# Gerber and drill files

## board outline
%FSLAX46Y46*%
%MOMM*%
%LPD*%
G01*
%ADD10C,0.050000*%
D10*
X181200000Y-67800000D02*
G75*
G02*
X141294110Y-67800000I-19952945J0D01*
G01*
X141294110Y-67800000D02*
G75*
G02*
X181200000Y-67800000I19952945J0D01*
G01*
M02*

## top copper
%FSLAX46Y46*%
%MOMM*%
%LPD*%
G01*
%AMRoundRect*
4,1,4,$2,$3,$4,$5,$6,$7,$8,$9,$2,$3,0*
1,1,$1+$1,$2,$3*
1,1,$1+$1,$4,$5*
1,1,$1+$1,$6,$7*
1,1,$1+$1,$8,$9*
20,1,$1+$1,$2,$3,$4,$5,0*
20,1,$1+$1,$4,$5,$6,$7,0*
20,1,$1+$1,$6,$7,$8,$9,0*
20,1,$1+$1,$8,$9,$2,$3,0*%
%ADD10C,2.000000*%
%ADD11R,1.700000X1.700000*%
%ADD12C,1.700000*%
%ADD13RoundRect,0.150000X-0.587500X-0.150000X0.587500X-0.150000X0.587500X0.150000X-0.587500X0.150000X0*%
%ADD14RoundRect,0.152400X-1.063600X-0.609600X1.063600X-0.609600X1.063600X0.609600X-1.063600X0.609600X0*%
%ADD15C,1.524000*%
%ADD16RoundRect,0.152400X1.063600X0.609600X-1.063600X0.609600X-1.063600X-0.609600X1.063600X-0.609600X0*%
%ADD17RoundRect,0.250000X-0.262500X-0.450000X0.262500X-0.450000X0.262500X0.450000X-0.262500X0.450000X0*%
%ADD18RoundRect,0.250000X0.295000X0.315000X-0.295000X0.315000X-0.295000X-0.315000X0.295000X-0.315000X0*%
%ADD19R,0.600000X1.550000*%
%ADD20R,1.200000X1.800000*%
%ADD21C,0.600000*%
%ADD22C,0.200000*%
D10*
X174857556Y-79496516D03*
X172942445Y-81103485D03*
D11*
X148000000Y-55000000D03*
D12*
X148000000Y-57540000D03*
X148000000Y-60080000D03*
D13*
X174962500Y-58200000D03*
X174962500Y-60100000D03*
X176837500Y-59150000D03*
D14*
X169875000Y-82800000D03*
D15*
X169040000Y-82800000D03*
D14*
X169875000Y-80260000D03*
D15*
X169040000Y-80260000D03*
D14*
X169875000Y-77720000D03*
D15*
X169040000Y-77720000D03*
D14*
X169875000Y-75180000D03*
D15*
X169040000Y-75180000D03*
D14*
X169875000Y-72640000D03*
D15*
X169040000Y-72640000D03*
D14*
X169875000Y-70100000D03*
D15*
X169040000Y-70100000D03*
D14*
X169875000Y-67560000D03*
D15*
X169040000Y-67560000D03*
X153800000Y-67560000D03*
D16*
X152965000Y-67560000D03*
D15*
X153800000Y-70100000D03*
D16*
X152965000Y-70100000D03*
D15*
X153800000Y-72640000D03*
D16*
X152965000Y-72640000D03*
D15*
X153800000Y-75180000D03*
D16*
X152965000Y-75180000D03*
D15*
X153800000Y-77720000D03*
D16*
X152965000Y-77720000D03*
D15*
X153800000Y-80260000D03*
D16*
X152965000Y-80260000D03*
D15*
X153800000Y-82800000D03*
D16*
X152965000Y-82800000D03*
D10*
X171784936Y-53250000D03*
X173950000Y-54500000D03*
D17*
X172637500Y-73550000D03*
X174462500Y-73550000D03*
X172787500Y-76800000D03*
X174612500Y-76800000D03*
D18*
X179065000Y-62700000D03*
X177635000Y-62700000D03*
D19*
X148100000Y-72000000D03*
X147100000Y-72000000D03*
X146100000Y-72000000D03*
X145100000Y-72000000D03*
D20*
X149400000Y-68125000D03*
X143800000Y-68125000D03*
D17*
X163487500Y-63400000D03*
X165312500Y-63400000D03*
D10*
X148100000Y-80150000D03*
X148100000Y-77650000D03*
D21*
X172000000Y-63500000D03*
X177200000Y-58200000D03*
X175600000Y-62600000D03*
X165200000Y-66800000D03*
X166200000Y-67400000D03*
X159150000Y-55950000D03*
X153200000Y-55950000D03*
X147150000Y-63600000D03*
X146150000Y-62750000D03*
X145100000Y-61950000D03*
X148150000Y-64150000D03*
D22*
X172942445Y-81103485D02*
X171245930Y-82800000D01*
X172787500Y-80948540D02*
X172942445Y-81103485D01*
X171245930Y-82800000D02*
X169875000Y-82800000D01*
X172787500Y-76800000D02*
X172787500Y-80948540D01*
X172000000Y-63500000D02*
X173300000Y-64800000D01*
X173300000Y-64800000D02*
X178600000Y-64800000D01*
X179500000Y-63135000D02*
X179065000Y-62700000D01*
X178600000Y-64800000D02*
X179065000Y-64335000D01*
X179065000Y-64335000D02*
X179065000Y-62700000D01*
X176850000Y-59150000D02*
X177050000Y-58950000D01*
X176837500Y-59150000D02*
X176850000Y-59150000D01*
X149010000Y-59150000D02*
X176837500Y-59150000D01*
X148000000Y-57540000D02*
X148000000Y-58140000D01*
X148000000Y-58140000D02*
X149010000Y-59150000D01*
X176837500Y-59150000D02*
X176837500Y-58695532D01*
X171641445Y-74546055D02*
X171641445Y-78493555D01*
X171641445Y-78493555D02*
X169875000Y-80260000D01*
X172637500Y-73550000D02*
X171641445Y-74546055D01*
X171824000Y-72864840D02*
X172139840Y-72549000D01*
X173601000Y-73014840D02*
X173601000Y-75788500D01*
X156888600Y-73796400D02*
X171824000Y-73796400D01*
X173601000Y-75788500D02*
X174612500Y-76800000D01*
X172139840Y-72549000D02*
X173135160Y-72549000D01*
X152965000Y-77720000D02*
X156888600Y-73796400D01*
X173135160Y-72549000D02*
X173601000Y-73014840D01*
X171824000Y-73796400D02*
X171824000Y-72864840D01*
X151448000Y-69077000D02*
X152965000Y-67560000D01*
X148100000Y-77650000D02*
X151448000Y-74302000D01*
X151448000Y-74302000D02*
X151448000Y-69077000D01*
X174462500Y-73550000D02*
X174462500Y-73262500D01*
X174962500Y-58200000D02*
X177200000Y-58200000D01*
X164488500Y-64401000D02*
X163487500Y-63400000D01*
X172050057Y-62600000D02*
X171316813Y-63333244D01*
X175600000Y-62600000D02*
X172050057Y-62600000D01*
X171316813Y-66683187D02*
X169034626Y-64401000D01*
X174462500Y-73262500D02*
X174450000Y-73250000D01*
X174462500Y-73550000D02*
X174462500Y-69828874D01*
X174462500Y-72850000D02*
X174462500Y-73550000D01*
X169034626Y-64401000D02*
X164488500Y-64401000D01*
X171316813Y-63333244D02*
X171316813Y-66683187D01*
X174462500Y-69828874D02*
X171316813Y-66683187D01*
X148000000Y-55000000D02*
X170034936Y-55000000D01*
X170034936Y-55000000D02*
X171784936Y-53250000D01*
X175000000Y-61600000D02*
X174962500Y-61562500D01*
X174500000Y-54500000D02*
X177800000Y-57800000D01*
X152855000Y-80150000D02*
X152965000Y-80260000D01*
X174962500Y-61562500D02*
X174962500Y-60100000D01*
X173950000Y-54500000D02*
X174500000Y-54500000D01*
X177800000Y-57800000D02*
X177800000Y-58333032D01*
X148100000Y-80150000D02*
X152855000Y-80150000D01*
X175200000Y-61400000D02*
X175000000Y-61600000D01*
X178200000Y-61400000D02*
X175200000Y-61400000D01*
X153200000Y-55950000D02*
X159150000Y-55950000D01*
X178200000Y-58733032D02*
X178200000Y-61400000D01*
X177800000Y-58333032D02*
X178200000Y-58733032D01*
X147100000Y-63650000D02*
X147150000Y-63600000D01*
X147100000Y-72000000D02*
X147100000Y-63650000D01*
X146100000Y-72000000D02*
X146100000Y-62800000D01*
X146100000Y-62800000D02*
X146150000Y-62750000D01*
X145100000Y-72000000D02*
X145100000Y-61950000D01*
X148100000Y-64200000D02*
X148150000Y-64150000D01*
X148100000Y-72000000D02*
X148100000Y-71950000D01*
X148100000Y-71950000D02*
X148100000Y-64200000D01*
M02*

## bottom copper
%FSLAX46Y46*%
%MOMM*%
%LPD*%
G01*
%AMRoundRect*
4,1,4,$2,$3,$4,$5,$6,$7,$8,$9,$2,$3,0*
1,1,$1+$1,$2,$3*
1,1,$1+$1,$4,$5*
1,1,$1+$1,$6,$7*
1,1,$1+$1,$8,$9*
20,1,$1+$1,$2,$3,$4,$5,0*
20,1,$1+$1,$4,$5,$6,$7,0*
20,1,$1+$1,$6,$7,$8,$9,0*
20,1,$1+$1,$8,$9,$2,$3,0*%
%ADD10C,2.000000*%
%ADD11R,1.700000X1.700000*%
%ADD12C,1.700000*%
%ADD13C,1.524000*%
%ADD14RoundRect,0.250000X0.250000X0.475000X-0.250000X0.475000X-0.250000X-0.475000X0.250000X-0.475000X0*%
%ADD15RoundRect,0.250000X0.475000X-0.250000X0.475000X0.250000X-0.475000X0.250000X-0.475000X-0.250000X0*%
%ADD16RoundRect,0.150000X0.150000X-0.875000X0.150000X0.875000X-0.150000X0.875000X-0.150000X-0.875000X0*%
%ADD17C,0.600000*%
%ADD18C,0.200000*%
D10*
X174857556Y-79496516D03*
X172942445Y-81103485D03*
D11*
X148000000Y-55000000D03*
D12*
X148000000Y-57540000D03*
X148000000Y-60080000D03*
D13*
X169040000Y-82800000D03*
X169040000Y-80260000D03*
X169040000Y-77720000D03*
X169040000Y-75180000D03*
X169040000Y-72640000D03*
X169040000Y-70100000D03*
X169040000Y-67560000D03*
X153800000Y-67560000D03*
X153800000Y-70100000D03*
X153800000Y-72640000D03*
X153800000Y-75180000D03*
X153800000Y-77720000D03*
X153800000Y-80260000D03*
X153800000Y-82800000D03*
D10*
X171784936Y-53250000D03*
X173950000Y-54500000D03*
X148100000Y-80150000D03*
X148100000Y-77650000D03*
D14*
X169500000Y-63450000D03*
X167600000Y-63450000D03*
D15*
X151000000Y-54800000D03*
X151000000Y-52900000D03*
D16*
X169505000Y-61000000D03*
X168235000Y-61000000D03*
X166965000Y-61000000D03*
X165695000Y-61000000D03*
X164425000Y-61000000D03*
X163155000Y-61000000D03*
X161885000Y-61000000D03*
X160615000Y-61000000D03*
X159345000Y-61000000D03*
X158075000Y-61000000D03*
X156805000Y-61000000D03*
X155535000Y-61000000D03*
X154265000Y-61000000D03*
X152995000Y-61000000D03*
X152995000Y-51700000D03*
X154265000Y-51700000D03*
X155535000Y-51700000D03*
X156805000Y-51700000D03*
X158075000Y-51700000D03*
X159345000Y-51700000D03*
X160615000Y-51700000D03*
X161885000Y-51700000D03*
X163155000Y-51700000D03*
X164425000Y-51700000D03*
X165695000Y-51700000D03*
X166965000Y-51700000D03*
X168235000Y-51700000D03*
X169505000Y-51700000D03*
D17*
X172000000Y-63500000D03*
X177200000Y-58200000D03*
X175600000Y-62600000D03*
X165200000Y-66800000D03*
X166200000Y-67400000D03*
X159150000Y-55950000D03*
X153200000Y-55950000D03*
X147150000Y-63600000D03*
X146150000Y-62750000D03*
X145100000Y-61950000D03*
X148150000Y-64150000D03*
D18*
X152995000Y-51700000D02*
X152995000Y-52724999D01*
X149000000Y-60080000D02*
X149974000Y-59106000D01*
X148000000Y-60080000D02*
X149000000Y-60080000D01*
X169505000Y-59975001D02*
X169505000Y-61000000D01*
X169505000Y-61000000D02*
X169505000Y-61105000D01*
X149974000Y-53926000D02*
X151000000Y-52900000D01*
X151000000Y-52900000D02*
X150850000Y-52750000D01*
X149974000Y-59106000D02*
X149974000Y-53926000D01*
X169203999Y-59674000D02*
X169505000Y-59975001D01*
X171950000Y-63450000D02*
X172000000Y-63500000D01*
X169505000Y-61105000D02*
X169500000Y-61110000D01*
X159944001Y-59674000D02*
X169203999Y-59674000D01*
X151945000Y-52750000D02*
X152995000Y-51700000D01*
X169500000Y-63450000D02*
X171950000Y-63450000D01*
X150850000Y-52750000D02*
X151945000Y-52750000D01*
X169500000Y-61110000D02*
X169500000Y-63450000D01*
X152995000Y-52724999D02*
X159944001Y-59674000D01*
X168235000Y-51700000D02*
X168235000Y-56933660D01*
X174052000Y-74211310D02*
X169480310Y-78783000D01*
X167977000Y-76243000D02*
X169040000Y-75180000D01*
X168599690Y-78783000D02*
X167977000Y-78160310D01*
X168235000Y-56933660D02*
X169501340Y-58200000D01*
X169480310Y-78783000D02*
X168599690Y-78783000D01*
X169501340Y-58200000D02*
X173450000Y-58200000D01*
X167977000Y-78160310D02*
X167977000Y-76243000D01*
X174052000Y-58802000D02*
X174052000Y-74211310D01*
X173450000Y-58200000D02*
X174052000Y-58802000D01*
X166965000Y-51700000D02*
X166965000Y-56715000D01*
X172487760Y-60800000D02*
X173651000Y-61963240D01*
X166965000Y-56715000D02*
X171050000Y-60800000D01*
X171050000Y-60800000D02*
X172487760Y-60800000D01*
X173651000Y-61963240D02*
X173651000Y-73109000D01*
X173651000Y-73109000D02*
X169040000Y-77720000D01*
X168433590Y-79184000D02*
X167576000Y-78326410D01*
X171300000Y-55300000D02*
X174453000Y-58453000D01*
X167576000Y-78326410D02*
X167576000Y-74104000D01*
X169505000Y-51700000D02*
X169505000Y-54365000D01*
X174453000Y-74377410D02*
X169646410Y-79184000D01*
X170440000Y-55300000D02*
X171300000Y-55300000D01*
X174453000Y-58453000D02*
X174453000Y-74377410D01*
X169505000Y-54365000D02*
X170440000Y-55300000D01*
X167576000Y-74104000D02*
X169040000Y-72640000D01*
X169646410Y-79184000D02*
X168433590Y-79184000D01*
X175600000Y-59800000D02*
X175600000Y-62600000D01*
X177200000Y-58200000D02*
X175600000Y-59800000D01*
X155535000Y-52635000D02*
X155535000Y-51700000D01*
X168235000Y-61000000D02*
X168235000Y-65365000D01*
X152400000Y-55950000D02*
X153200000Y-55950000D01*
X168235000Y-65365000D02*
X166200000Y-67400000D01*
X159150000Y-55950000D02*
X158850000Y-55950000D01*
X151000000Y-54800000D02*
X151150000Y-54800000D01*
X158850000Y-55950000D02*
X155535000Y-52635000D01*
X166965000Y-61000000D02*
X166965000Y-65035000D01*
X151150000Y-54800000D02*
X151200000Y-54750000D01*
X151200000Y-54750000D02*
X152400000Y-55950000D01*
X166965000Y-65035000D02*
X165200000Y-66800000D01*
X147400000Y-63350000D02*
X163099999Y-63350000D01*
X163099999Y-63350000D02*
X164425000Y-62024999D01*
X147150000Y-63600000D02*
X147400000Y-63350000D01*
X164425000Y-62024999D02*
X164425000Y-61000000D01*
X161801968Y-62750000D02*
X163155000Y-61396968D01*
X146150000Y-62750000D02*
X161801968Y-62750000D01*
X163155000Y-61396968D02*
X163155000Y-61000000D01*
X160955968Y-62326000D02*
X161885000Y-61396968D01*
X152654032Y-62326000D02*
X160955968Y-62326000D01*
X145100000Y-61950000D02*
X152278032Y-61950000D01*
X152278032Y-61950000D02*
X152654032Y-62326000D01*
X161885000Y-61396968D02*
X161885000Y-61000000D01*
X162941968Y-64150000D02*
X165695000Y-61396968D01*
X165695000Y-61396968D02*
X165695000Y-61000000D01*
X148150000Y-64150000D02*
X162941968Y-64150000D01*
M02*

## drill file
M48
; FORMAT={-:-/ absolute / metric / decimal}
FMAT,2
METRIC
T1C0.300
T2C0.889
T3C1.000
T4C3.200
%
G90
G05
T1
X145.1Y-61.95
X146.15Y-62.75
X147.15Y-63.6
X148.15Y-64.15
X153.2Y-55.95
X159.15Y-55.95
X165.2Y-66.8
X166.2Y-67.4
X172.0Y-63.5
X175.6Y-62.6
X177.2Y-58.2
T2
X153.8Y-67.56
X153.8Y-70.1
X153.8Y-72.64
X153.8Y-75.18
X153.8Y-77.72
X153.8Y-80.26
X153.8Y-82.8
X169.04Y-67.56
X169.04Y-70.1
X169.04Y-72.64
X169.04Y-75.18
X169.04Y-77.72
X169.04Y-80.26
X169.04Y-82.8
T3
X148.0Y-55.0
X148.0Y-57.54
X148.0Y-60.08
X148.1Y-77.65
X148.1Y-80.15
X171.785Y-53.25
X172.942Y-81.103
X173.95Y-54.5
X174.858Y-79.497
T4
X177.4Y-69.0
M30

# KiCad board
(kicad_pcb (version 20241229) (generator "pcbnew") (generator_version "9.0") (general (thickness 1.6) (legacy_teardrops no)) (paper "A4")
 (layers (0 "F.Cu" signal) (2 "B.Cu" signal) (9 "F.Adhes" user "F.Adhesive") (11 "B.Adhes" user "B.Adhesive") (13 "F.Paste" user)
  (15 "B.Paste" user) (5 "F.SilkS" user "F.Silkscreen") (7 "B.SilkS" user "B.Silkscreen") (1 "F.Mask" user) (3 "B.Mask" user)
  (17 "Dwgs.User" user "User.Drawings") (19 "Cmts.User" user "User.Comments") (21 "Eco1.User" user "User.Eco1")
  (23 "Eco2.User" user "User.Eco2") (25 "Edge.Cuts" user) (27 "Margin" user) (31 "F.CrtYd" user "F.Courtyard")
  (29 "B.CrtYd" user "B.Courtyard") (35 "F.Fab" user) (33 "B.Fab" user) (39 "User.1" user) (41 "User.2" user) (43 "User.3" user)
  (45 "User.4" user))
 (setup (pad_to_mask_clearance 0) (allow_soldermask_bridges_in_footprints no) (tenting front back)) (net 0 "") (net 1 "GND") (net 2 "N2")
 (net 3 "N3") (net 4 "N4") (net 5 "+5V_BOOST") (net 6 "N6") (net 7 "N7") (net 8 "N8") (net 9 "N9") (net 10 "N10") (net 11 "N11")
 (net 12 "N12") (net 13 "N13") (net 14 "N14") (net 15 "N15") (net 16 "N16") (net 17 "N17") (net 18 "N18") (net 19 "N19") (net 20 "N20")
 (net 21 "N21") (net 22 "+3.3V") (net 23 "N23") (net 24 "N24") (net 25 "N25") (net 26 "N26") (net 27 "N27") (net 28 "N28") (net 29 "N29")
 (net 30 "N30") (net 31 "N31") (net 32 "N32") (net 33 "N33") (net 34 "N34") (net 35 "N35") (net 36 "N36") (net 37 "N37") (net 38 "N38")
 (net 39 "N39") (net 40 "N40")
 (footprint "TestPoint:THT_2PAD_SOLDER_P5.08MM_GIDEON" (layer "F.Cu") (at 174.857556 79.496516 -140)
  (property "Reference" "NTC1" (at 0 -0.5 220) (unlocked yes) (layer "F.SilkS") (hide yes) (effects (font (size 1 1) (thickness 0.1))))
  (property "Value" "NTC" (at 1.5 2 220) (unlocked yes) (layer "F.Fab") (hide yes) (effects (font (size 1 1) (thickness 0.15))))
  (pad "1" thru_hole circle (at 0 0 220) (size 2 2) (drill 1) (layers "*.Cu" "*.Mask") (remove_unused_layers no) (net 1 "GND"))
  (pad "2" thru_hole circle (at 2.5 0 220) (size 2 2) (drill 1) (layers "*.Cu" "*.Mask") (remove_unused_layers no) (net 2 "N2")))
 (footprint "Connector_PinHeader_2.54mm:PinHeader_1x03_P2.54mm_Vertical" (layer "F.Cu") (at 148 55)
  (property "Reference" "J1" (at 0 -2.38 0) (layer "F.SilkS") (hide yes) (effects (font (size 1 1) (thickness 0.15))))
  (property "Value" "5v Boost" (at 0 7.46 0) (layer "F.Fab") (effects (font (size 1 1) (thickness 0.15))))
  (pad "1" thru_hole rect (at 0 0) (size 1.7 1.7) (drill 1) (layers "*.Cu" "*.Mask") (remove_unused_layers no) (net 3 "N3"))
  (pad "2" thru_hole circle (at 0 2.54) (size 1.7 1.7) (drill 1) (layers "*.Cu" "*.Mask") (remove_unused_layers no) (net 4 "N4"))
  (pad "3" thru_hole circle (at 0 5.08) (size 1.7 1.7) (drill 1) (layers "*.Cu" "*.Mask") (remove_unused_layers no) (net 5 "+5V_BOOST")))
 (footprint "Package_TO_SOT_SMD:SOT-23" (layer "F.Cu") (at 175.9 59.15)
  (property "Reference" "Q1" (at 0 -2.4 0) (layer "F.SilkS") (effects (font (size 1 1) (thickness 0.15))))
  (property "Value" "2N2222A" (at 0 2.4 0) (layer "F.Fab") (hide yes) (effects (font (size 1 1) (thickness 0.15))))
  (pad "1" smd roundrect (at -0.9375 -0.95) (size 1.475 0.6) (layers "F.Cu" "F.Mask" "F.Paste") (roundrect_rratio 0.25) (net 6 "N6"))
  (pad "2" smd roundrect (at -0.9375 0.95) (size 1.475 0.6) (layers "F.Cu" "F.Mask" "F.Paste") (roundrect_rratio 0.25) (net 1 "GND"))
  (pad "3" smd roundrect (at 0.9375 0) (size 1.475 0.6) (layers "F.Cu" "F.Mask" "F.Paste") (roundrect_rratio 0.25) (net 4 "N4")))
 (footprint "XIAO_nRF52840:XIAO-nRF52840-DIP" (layer "F.Cu") (at 161.42 75.18 180)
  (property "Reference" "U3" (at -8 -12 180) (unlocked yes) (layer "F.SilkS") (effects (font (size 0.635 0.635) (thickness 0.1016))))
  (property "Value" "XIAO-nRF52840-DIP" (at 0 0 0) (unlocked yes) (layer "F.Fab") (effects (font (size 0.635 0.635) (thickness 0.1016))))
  (pad "1" smd roundrect (at -8.455 -7.62) (size 2.432 1.524) (layers "F.Cu" "F.Mask") (roundrect_rratio 0.1) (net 2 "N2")
   (thermal_bridge_angle 45))
  (pad "1" thru_hole circle (at -7.62 -7.62) (size 1.524 1.524) (drill 0.889) (layers "*.Cu" "*.Mask") (remove_unused_layers no)
   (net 2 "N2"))
  (pad "2" smd roundrect (at -8.455 -5.08) (size 2.432 1.524) (layers "F.Cu" "F.Mask") (roundrect_rratio 0.1) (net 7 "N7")
   (thermal_bridge_angle 45))
  (pad "2" thru_hole circle (at -7.62 -5.08) (size 1.524 1.524) (drill 0.889) (layers "*.Cu" "*.Mask") (remove_unused_layers no)
   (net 7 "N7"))
  (pad "3" smd roundrect (at -8.455 -2.54) (size 2.432 1.524) (layers "F.Cu" "F.Mask") (roundrect_rratio 0.1) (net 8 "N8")
   (thermal_bridge_angle 45))
  (pad "3" thru_hole circle (at -7.62 -2.54) (size 1.524 1.524) (drill 0.889) (layers "*.Cu" "*.Mask") (remove_unused_layers no)
   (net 8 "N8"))
  (pad "4" smd roundrect (at -8.455 0) (size 2.432 1.524) (layers "F.Cu" "F.Mask") (roundrect_rratio 0.1) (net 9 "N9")
   (thermal_bridge_angle 45))
  (pad "4" thru_hole circle (at -7.62 0) (size 1.524 1.524) (drill 0.889) (layers "*.Cu" "*.Mask") (remove_unused_layers no) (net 9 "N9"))
  (pad "5" smd roundrect (at -8.455 2.54) (size 2.432 1.524) (layers "F.Cu" "F.Mask") (roundrect_rratio 0.1) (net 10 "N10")
   (thermal_bridge_angle 45))
  (pad "5" thru_hole circle (at -7.62 2.54) (size 1.524 1.524) (drill 0.889) (layers "*.Cu" "*.Mask") (remove_unused_layers no)
   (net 10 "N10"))
  (pad "6" smd roundrect (at -8.455 5.08) (size 2.432 1.524) (layers "F.Cu" "F.Mask") (roundrect_rratio 0.1) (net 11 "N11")
   (thermal_bridge_angle 45))
  (pad "6" thru_hole circle (at -7.62 5.08) (size 1.524 1.524) (drill 0.889) (layers "*.Cu" "*.Mask") (remove_unused_layers no)
   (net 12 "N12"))
  (pad "7" smd roundrect (at -8.455 7.62) (size 2.432 1.524) (layers "F.Cu" "F.Mask") (roundrect_rratio 0.1) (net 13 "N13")
   (thermal_bridge_angle 45))
  (pad "7" thru_hole circle (at -7.62 7.62) (size 1.524 1.524) (drill 0.889) (layers "*.Cu" "*.Mask") (remove_unused_layers no)
   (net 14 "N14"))
  (pad "8" thru_hole circle (at 7.62 7.62 180) (size 1.524 1.524) (drill 0.889) (layers "*.Cu" "*.Mask") (remove_unused_layers no)
   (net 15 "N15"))
  (pad "8" smd roundrect (at 8.455 7.62 180) (size 2.432 1.524) (layers "F.Cu" "F.Mask") (roundrect_rratio 0.1) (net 15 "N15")
   (thermal_bridge_angle 45))
  (pad "9" thru_hole circle (at 7.62 5.08 180) (size 1.524 1.524) (drill 0.889) (layers "*.Cu" "*.Mask") (remove_unused_layers no)
   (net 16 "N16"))
  (pad "9" smd roundrect (at 8.455 5.08 180) (size 2.432 1.524) (layers "F.Cu" "F.Mask") (roundrect_rratio 0.1) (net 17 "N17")
   (thermal_bridge_angle 45))
  (pad "10" thru_hole circle (at 7.62 2.54 180) (size 1.524 1.524) (drill 0.889) (layers "*.Cu" "*.Mask") (remove_unused_layers no)
   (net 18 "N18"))
  (pad "10" smd roundrect (at 8.455 2.54 180) (size 2.432 1.524) (layers "F.Cu" "F.Mask") (roundrect_rratio 0.1) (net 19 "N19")
   (thermal_bridge_angle 45))
  (pad "11" thru_hole circle (at 7.62 0 180) (size 1.524 1.524) (drill 0.889) (layers "*.Cu" "*.Mask") (remove_unused_layers no)
   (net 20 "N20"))
  (pad "11" smd roundrect (at 8.455 0 180) (size 2.432 1.524) (layers "F.Cu" "F.Mask") (roundrect_rratio 0.1) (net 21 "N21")
   (thermal_bridge_angle 45))
  (pad "12" thru_hole circle (at 7.62 -2.54 180) (size 1.524 1.524) (drill 0.889) (layers "*.Cu" "*.Mask") (remove_unused_layers no)
   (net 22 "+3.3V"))
  (pad "12" smd roundrect (at 8.455 -2.54 180) (size 2.432 1.524) (layers "F.Cu" "F.Mask") (roundrect_rratio 0.1) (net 22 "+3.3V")
   (thermal_bridge_angle 45))
  (pad "13" thru_hole circle (at 7.62 -5.08 180) (size 1.524 1.524) (drill 0.889) (layers "*.Cu" "*.Mask") (remove_unused_layers no)
   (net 1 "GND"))
  (pad "13" smd roundrect (at 8.455 -5.08 180) (size 2.432 1.524) (layers "F.Cu" "F.Mask") (roundrect_rratio 0.1) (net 1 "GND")
   (thermal_bridge_angle 45))
  (pad "14" thru_hole circle (at 7.62 -7.62 180) (size 1.524 1.524) (drill 0.889) (layers "*.Cu" "*.Mask") (remove_unused_layers no)
   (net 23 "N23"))
  (pad "14" smd roundrect (at 8.455 -7.62 180) (size 2.432 1.524) (layers "F.Cu" "F.Mask") (roundrect_rratio 0.1) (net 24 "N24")
   (thermal_bridge_angle 45)))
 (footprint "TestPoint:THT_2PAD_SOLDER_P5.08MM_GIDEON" (layer "F.Cu") (at 171.784936 53.25 -30)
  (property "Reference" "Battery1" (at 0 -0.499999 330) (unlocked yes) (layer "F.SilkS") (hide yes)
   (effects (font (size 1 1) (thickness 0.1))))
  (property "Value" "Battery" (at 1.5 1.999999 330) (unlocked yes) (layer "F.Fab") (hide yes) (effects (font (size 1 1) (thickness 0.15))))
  (pad "1" thru_hole circle (at 0 0 330) (size 2 2) (drill 1) (layers "*.Cu" "*.Mask") (remove_unused_layers no) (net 3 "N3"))
  (pad "2" thru_hole circle (at 2.5 0 330) (size 2 2) (drill 1) (layers "*.Cu" "*.Mask") (remove_unused_layers no) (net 1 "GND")))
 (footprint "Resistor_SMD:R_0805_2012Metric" (layer "F.Cu") (at 173.55 73.55)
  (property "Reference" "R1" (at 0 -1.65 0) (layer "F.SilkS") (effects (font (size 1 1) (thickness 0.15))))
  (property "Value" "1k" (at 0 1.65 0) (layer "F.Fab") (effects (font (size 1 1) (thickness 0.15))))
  (pad "1" smd roundrect (at -0.9125 0) (size 1.025 1.4) (layers "F.Cu" "F.Mask" "F.Paste") (roundrect_rratio 0.243902) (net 7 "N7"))
  (pad "2" smd roundrect (at 0.9125 0) (size 1.025 1.4) (layers "F.Cu" "F.Mask" "F.Paste") (roundrect_rratio 0.243902) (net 6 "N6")))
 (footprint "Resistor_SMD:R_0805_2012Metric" (layer "F.Cu") (at 173.7 76.8)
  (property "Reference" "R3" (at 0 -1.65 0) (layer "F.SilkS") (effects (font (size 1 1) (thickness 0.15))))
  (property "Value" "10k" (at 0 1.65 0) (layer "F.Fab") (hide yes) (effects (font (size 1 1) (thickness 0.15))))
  (pad "1" smd roundrect (at -0.9125 0) (size 1.025 1.4) (layers "F.Cu" "F.Mask" "F.Paste") (roundrect_rratio 0.243902) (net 2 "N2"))
  (pad "2" smd roundrect (at 0.9125 0) (size 1.025 1.4) (layers "F.Cu" "F.Mask" "F.Paste") (roundrect_rratio 0.243902) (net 22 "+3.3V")))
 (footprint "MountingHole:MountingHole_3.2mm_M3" (layer "F.Cu") (at 177.4 69)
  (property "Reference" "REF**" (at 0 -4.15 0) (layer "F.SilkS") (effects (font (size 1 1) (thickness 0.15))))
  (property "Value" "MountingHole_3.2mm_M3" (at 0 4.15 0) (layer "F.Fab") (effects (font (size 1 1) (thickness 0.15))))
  (pad "" np_thru_hole circle (at 0 0) (size 3.2 3.2) (drill 3.2) (layers "*.Cu" "*.Mask")))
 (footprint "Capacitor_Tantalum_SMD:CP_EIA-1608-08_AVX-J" (layer "F.Cu") (at 178.35 62.7 180)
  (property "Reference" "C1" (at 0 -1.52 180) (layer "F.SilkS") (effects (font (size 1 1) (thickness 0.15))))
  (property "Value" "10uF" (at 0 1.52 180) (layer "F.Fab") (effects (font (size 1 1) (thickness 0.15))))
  (pad "1" smd roundrect (at -0.715 0 180) (size 1.09 1.13) (layers "F.Cu" "F.Mask" "F.Paste") (roundrect_rratio 0.229358)
   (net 5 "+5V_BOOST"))
  (pad "2" smd roundrect (at 0.715 0 180) (size 1.09 1.13) (layers "F.Cu" "F.Mask" "F.Paste") (roundrect_rratio 0.229358) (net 1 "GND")))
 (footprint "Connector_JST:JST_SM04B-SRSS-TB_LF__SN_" (layer "F.Cu") (at 146.6 72 180)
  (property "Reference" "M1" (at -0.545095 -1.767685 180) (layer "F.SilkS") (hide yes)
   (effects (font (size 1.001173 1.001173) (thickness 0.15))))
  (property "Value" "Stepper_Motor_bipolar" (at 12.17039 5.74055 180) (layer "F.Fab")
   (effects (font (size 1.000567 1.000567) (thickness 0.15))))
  (pad "1" smd rect (at -1.5 0 180) (size 0.6 1.55) (layers "F.Cu" "F.Mask" "F.Paste") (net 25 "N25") (solder_mask_margin 0.102))
  (pad "2" smd rect (at -0.5 0 180) (size 0.6 1.55) (layers "F.Cu" "F.Mask" "F.Paste") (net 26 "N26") (solder_mask_margin 0.102))
  (pad "3" smd rect (at 0.5 0 180) (size 0.6 1.55) (layers "F.Cu" "F.Mask" "F.Paste") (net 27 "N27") (solder_mask_margin 0.102))
  (pad "4" smd rect (at 1.5 0 180) (size 0.6 1.55) (layers "F.Cu" "F.Mask" "F.Paste") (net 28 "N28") (solder_mask_margin 0.102))
  (pad "S1" smd rect (at -2.8 3.875 180) (size 1.2 1.8) (layers "F.Cu" "F.Mask" "F.Paste") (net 1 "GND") (solder_mask_margin 0.102))
  (pad "S2" smd rect (at 2.8 3.875 180) (size 1.2 1.8) (layers "F.Cu" "F.Mask" "F.Paste") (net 1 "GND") (solder_mask_margin 0.102)))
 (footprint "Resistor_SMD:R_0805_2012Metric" (layer "F.Cu") (at 164.4 63.4)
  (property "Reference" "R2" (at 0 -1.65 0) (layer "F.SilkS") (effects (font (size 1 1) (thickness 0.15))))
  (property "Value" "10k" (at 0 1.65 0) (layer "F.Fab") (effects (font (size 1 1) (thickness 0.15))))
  (pad "1" smd roundrect (at -0.9125 0) (size 1.025 1.4) (layers "F.Cu" "F.Mask" "F.Paste") (roundrect_rratio 0.243902) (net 6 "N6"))
  (pad "2" smd roundrect (at 0.9125 0) (size 1.025 1.4) (layers "F.Cu" "F.Mask" "F.Paste") (roundrect_rratio 0.243902) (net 1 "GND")))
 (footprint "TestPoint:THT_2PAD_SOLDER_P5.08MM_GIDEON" (layer "F.Cu") (at 148.1 80.15 90)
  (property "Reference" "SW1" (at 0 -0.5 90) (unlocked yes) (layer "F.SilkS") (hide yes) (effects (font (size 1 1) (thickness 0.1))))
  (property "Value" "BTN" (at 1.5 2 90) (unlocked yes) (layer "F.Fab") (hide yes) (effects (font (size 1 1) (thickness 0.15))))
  (pad "1" thru_hole circle (at 0 0 90) (size 2 2) (drill 1) (layers "*.Cu" "*.Mask") (remove_unused_layers no) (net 1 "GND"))
  (pad "2" thru_hole circle (at 2.5 0 90) (size 2 2) (drill 1) (layers "*.Cu" "*.Mask") (remove_unused_layers no) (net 15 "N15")))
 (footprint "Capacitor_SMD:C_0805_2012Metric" (layer "B.Cu") (at 168.55 63.45 180)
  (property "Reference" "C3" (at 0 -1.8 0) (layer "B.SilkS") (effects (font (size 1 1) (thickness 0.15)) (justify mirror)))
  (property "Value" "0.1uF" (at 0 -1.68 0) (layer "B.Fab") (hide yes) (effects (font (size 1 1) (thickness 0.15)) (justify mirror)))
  (pad "1" smd roundrect (at -0.95 0 180) (size 1 1.45) (layers "B.Cu" "B.Mask" "B.Paste") (roundrect_rratio 0.25) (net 5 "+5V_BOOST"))
  (pad "2" smd roundrect (at 0.95 0 180) (size 1 1.45) (layers "B.Cu" "B.Mask" "B.Paste") (roundrect_rratio 0.25) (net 1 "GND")))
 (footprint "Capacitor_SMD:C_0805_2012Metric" (layer "B.Cu") (at 151 53.85 90)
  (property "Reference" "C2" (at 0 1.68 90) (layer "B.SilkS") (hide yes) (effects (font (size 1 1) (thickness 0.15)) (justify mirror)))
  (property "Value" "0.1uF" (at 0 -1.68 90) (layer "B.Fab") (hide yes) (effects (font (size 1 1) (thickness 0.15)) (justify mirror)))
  (pad "1" smd roundrect (at -0.95 0 90) (size 1 1.45) (layers "B.Cu" "B.Mask" "B.Paste") (roundrect_rratio 0.25) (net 1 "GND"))
  (pad "2" smd roundrect (at 0.95 0 90) (size 1 1.45) (layers "B.Cu" "B.Mask" "B.Paste") (roundrect_rratio 0.25) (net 5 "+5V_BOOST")))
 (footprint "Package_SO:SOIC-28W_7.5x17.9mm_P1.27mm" (layer "B.Cu") (at 161.25 56.35 90)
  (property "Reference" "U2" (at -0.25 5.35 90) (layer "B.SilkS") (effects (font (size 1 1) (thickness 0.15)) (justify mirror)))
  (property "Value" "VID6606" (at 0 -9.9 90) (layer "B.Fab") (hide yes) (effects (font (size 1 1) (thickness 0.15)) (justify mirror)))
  (pad "1" smd roundrect (at -4.65 8.255 90) (size 2.05 0.6) (layers "B.Cu" "B.Mask" "B.Paste") (roundrect_rratio 0.25) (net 5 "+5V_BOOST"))
  (pad "2" smd roundrect (at -4.65 6.985 90) (size 2.05 0.6) (layers "B.Cu" "B.Mask" "B.Paste") (roundrect_rratio 0.25) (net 1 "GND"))
  (pad "3" smd roundrect (at -4.65 5.715 90) (size 2.05 0.6) (layers "B.Cu" "B.Mask" "B.Paste") (roundrect_rratio 0.25) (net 1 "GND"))
  (pad "4" smd roundrect (at -4.65 4.445 90) (size 2.05 0.6) (layers "B.Cu" "B.Mask" "B.Paste") (roundrect_rratio 0.25) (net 25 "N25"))
  (pad "5" smd roundrect (at -4.65 3.175 90) (size 2.05 0.6) (layers "B.Cu" "B.Mask" "B.Paste") (roundrect_rratio 0.25) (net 26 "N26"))
  (pad "6" smd roundrect (at -4.65 1.905 90) (size 2.05 0.6) (layers "B.Cu" "B.Mask" "B.Paste") (roundrect_rratio 0.25) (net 27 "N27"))
  (pad "7" smd roundrect (at -4.65 0.635 90) (size 2.05 0.6) (layers "B.Cu" "B.Mask" "B.Paste") (roundrect_rratio 0.25) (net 28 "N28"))
  (pad "8" smd roundrect (at -4.65 -0.635 90) (size 2.05 0.6) (layers "B.Cu" "B.Mask" "B.Paste") (roundrect_rratio 0.25) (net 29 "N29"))
  (pad "9" smd roundrect (at -4.65 -1.905 90) (size 2.05 0.6) (layers "B.Cu" "B.Mask" "B.Paste") (roundrect_rratio 0.25) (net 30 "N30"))
  (pad "10" smd roundrect (at -4.65 -3.175 90) (size 2.05 0.6) (layers "B.Cu" "B.Mask" "B.Paste") (roundrect_rratio 0.25) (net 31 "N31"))
  (pad "11" smd roundrect (at -4.65 -4.445 90) (size 2.05 0.6) (layers "B.Cu" "B.Mask" "B.Paste") (roundrect_rratio 0.25) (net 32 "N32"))
  (pad "12" smd roundrect (at -4.65 -5.715 90) (size 2.05 0.6) (layers "B.Cu" "B.Mask" "B.Paste") (roundrect_rratio 0.25) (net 1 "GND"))
  (pad "13" smd roundrect (at -4.65 -6.985 90) (size 2.05 0.6) (layers "B.Cu" "B.Mask" "B.Paste") (roundrect_rratio 0.25) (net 1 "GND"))
  (pad "14" smd roundrect (at -4.65 -8.255 90) (size 2.05 0.6) (layers "B.Cu" "B.Mask" "B.Paste") (roundrect_rratio 0.25) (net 1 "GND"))
  (pad "15" smd roundrect (at 4.65 -8.255 90) (size 2.05 0.6) (layers "B.Cu" "B.Mask" "B.Paste") (roundrect_rratio 0.25) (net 5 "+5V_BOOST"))
  (pad "16" smd roundrect (at 4.65 -6.985 90) (size 2.05 0.6) (layers "B.Cu" "B.Mask" "B.Paste") (roundrect_rratio 0.25) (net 1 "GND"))
  (pad "17" smd roundrect (at 4.65 -5.715 90) (size 2.05 0.6) (layers "B.Cu" "B.Mask" "B.Paste") (roundrect_rratio 0.25) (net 1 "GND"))
  (pad "18" smd roundrect (at 4.65 -4.445 90) (size 2.05 0.6) (layers "B.Cu" "B.Mask" "B.Paste") (roundrect_rratio 0.25) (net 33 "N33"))
  (pad "19" smd roundrect (at 4.65 -3.175 90) (size 2.05 0.6) (layers "B.Cu" "B.Mask" "B.Paste") (roundrect_rratio 0.25) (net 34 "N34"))
  (pad "20" smd roundrect (at 4.65 -1.905 90) (size 2.05 0.6) (layers "B.Cu" "B.Mask" "B.Paste") (roundrect_rratio 0.25) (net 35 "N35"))
  (pad "21" smd roundrect (at 4.65 -0.635 90) (size 2.05 0.6) (layers "B.Cu" "B.Mask" "B.Paste") (roundrect_rratio 0.25) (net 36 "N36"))
  (pad "22" smd roundrect (at 4.65 0.635 90) (size 2.05 0.6) (layers "B.Cu" "B.Mask" "B.Paste") (roundrect_rratio 0.25) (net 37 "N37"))
  (pad "23" smd roundrect (at 4.65 1.905 90) (size 2.05 0.6) (layers "B.Cu" "B.Mask" "B.Paste") (roundrect_rratio 0.25) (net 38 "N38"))
  (pad "24" smd roundrect (at 4.65 3.175 90) (size 2.05 0.6) (layers "B.Cu" "B.Mask" "B.Paste") (roundrect_rratio 0.25) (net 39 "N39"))
  (pad "25" smd roundrect (at 4.65 4.445 90) (size 2.05 0.6) (layers "B.Cu" "B.Mask" "B.Paste") (roundrect_rratio 0.25) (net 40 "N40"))
  (pad "26" smd roundrect (at 4.65 5.715 90) (size 2.05 0.6) (layers "B.Cu" "B.Mask" "B.Paste") (roundrect_rratio 0.25) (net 8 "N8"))
  (pad "27" smd roundrect (at 4.65 6.985 90) (size 2.05 0.6) (layers "B.Cu" "B.Mask" "B.Paste") (roundrect_rratio 0.25) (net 9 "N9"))
  (pad "28" smd roundrect (at 4.65 8.255 90) (size 2.05 0.6) (layers "B.Cu" "B.Mask" "B.Paste") (roundrect_rratio 0.25) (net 10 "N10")))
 (gr_circle (center 161.247055 67.8) (end 175.847055 81.4) (stroke (width 0.05) (type default)) (fill no) (layer "Edge.Cuts"))
 (segment (start 172.942445 81.103485) (end 171.24593 82.8) (width 0.2) (layer "F.Cu") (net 2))
 (segment (start 172.7875 80.94854) (end 172.942445 81.103485) (width 0.2) (layer "F.Cu") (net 2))
 (segment (start 171.24593 82.8) (end 169.875 82.8) (width 0.2) (layer "F.Cu") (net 2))
 (segment (start 172.7875 76.8) (end 172.7875 80.94854) (width 0.2) (layer "F.Cu") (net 2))
 (segment (start 172 63.5) (end 173.3 64.8) (width 0.2) (layer "F.Cu") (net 5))
 (segment (start 173.3 64.8) (end 178.6 64.8) (width 0.2) (layer "F.Cu") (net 5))
 (segment (start 179.5 63.135) (end 179.065 62.7) (width 0.2) (layer "F.Cu") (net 5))
 (segment (start 178.6 64.8) (end 179.065 64.335) (width 0.2) (layer "F.Cu") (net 5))
 (segment (start 179.065 64.335) (end 179.065 62.7) (width 0.2) (layer "F.Cu") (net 5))
 (via (at 172 63.5) (size 0.6) (drill 0.3) (layers "F.Cu" "B.Cu") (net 5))
 (segment (start 152.995 51.7) (end 152.995 52.724999) (width 0.2) (layer "B.Cu") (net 5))
 (segment (start 149 60.08) (end 149.974 59.106) (width 0.2) (layer "B.Cu") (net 5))
 (segment (start 148 60.08) (end 149 60.08) (width 0.2) (layer "B.Cu") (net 5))
 (segment (start 169.505 59.975001) (end 169.505 61) (width 0.2) (layer "B.Cu") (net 5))
 (segment (start 169.505 61) (end 169.505 61.105) (width 0.2) (layer "B.Cu") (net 5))
 (segment (start 149.974 53.926) (end 151 52.9) (width 0.2) (layer "B.Cu") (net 5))
 (segment (start 151 52.9) (end 150.85 52.75) (width 0.2) (layer "B.Cu") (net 5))
 (segment (start 149.974 59.106) (end 149.974 53.926) (width 0.2) (layer "B.Cu") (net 5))
 (segment (start 169.203999 59.674) (end 169.505 59.975001) (width 0.2) (layer "B.Cu") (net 5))
 (segment (start 171.95 63.45) (end 172 63.5) (width 0.2) (layer "B.Cu") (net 5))
 (segment (start 169.505 61.105) (end 169.5 61.11) (width 0.2) (layer "B.Cu") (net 5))
 (segment (start 159.944001 59.674) (end 169.203999 59.674) (width 0.2) (layer "B.Cu") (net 5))
 (segment (start 151.945 52.75) (end 152.995 51.7) (width 0.2) (layer "B.Cu") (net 5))
 (segment (start 169.5 63.45) (end 171.95 63.45) (width 0.2) (layer "B.Cu") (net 5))
 (segment (start 150.85 52.75) (end 151.945 52.75) (width 0.2) (layer "B.Cu") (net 5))
 (segment (start 169.5 61.11) (end 169.5 63.45) (width 0.2) (layer "B.Cu") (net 5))
 (segment (start 152.995 52.724999) (end 159.944001 59.674) (width 0.2) (layer "B.Cu") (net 5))
 (segment (start 176.85 59.15) (end 177.05 58.95) (width 0.2) (layer "F.Cu") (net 4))
 (segment (start 176.8375 59.15) (end 176.85 59.15) (width 0.2) (layer "F.Cu") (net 4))
 (segment (start 149.01 59.15) (end 176.8375 59.15) (width 0.2) (layer "F.Cu") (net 4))
 (segment (start 148 57.54) (end 148 58.14) (width 0.2) (layer "F.Cu") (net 4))
 (segment (start 148 58.14) (end 149.01 59.15) (width 0.2) (layer "F.Cu") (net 4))
 (segment (start 176.8375 59.15) (end 176.8375 58.695532) (width 0.2) (layer "F.Cu") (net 4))
 (segment (start 171.641445 74.546055) (end 171.641445 78.493555) (width 0.2) (layer "F.Cu") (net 7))
 (segment (start 171.641445 78.493555) (end 169.875 80.26) (width 0.2) (layer "F.Cu") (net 7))
 (segment (start 172.6375 73.55) (end 171.641445 74.546055) (width 0.2) (layer "F.Cu") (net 7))
 (segment (start 168.235 51.7) (end 168.235 56.93366) (width 0.2) (layer "B.Cu") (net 9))
 (segment (start 174.052 74.21131) (end 169.48031 78.783) (width 0.2) (layer "B.Cu") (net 9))
 (segment (start 167.977 76.243) (end 169.04 75.18) (width 0.2) (layer "B.Cu") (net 9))
 (segment (start 168.59969 78.783) (end 167.977 78.16031) (width 0.2) (layer "B.Cu") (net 9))
 (segment (start 168.235 56.93366) (end 169.50134 58.2) (width 0.2) (layer "B.Cu") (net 9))
 (segment (start 169.48031 78.783) (end 168.59969 78.783) (width 0.2) (layer "B.Cu") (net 9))
 (segment (start 169.50134 58.2) (end 173.45 58.2) (width 0.2) (layer "B.Cu") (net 9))
 (segment (start 167.977 78.16031) (end 167.977 76.243) (width 0.2) (layer "B.Cu") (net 9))
 (segment (start 174.052 58.802) (end 174.052 74.21131) (width 0.2) (layer "B.Cu") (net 9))
 (segment (start 173.45 58.2) (end 174.052 58.802) (width 0.2) (layer "B.Cu") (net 9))
 (segment (start 171.824 72.86484) (end 172.13984 72.549) (width 0.2) (layer "F.Cu") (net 22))
 (segment (start 173.601 73.01484) (end 173.601 75.7885) (width 0.2) (layer "F.Cu") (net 22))
 (segment (start 156.8886 73.7964) (end 171.824 73.7964) (width 0.2) (layer "F.Cu") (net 22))
 (segment (start 173.601 75.7885) (end 174.6125 76.8) (width 0.2) (layer "F.Cu") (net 22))
 (segment (start 172.13984 72.549) (end 173.13516 72.549) (width 0.2) (layer "F.Cu") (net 22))
 (segment (start 152.965 77.72) (end 156.8886 73.7964) (width 0.2) (layer "F.Cu") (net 22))
 (segment (start 173.13516 72.549) (end 173.601 73.01484) (width 0.2) (layer "F.Cu") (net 22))
 (segment (start 171.824 73.7964) (end 171.824 72.86484) (width 0.2) (layer "F.Cu") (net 22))
 (segment (start 151.448 69.077) (end 152.965 67.56) (width 0.2) (layer "F.Cu") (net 15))
 (segment (start 148.1 77.65) (end 151.448 74.302) (width 0.2) (layer "F.Cu") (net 15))
 (segment (start 151.448 74.302) (end 151.448 69.077) (width 0.2) (layer "F.Cu") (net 15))
 (segment (start 166.965 51.7) (end 166.965 56.715) (width 0.2) (layer "B.Cu") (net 8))
 (segment (start 172.48776 60.8) (end 173.651 61.96324) (width 0.2) (layer "B.Cu") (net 8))
 (segment (start 166.965 56.715) (end 171.05 60.8) (width 0.2) (layer "B.Cu") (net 8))
 (segment (start 171.05 60.8) (end 172.48776 60.8) (width 0.2) (layer "B.Cu") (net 8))
 (segment (start 173.651 61.96324) (end 173.651 73.109) (width 0.2) (layer "B.Cu") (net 8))
 (segment (start 173.651 73.109) (end 169.04 77.72) (width 0.2) (layer "B.Cu") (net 8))
 (segment (start 168.43359 79.184) (end 167.576 78.32641) (width 0.2) (layer "B.Cu") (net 10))
 (segment (start 171.3 55.3) (end 174.453 58.453) (width 0.2) (layer "B.Cu") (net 10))
 (segment (start 167.576 78.32641) (end 167.576 74.104) (width 0.2) (layer "B.Cu") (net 10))
 (segment (start 169.505 51.7) (end 169.505 54.365) (width 0.2) (layer "B.Cu") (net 10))
 (segment (start 174.453 74.37741) (end 169.64641 79.184) (width 0.2) (layer "B.Cu") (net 10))
 (segment (start 170.44 55.3) (end 171.3 55.3) (width 0.2) (layer "B.Cu") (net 10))
 (segment (start 174.453 58.453) (end 174.453 74.37741) (width 0.2) (layer "B.Cu") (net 10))
 (segment (start 169.505 54.365) (end 170.44 55.3) (width 0.2) (layer "B.Cu") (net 10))
 (segment (start 167.576 74.104) (end 169.04 72.64) (width 0.2) (layer "B.Cu") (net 10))
 (segment (start 169.64641 79.184) (end 168.43359 79.184) (width 0.2) (layer "B.Cu") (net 10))
 (segment (start 174.4625 73.55) (end 174.4625 73.2625) (width 0.2) (layer "F.Cu") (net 6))
 (segment (start 174.9625 58.2) (end 177.2 58.2) (width 0.2) (layer "F.Cu") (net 6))
 (segment (start 164.4885 64.401) (end 163.4875 63.4) (width 0.2) (layer "F.Cu") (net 6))
 (segment (start 172.050057 62.6) (end 171.316813 63.333244) (width 0.2) (layer "F.Cu") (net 6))
 (segment (start 175.6 62.6) (end 172.050057 62.6) (width 0.2) (layer "F.Cu") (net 6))
 (segment (start 171.316813 66.683187) (end 169.034626 64.401) (width 0.2) (layer "F.Cu") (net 6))
 (segment (start 174.4625 73.2625) (end 174.45 73.25) (width 0.2) (layer "F.Cu") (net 6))
 (segment (start 174.4625 73.55) (end 174.4625 69.828874) (width 0.2) (layer "F.Cu") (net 6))
 (segment (start 174.4625 72.85) (end 174.4625 73.55) (width 0.2) (layer "F.Cu") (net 6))
 (segment (start 169.034626 64.401) (end 164.4885 64.401) (width 0.2) (layer "F.Cu") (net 6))
 (segment (start 171.316813 63.333244) (end 171.316813 66.683187) (width 0.2) (layer "F.Cu") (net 6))
 (segment (start 174.4625 69.828874) (end 171.316813 66.683187) (width 0.2) (layer "F.Cu") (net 6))
 (via (at 177.2 58.2) (size 0.6) (drill 0.3) (layers "F.Cu" "B.Cu") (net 6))
 (via (at 175.6 62.6) (size 0.6) (drill 0.3) (layers "F.Cu" "B.Cu") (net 6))
 (segment (start 175.6 59.8) (end 175.6 62.6) (width 0.2) (layer "B.Cu") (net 6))
 (segment (start 177.2 58.2) (end 175.6 59.8) (width 0.2) (layer "B.Cu") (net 6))
 (segment (start 148 55) (end 170.034936 55) (width 0.2) (layer "F.Cu") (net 3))
 (segment (start 170.034936 55) (end 171.784936 53.25) (width 0.2) (layer "F.Cu") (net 3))
 (segment (start 175 61.6) (end 174.9625 61.5625) (width 0.2) (layer "F.Cu") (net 1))
 (segment (start 174.5 54.5) (end 177.8 57.8) (width 0.2) (layer "F.Cu") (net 1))
 (segment (start 152.855 80.15) (end 152.965 80.26) (width 0.2) (layer "F.Cu") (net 1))
 (segment (start 174.9625 61.5625) (end 174.9625 60.1) (width 0.2) (layer "F.Cu") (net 1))
 (segment (start 173.95 54.5) (end 174.5 54.5) (width 0.2) (layer "F.Cu") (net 1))
 (segment (start 177.8 57.8) (end 177.8 58.333032) (width 0.2) (layer "F.Cu") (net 1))
 (segment (start 148.1 80.15) (end 152.855 80.15) (width 0.2) (layer "F.Cu") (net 1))
 (segment (start 175.2 61.4) (end 175 61.6) (width 0.2) (layer "F.Cu") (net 1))
 (segment (start 178.2 61.4) (end 175.2 61.4) (width 0.2) (layer "F.Cu") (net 1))
 (segment (start 153.2 55.95) (end 159.15 55.95) (width 0.2) (layer "F.Cu") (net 1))
 (segment (start 178.2 58.733032) (end 178.2 61.4) (width 0.2) (layer "F.Cu") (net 1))
 (segment (start 177.8 58.333032) (end 178.2 58.733032) (width 0.2) (layer "F.Cu") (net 1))
 (via (at 165.2 66.8) (size 0.6) (drill 0.3) (layers "F.Cu" "B.Cu") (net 1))
 (via (at 166.2 67.4) (size 0.6) (drill 0.3) (layers "F.Cu" "B.Cu") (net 1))
 (via (at 159.15 55.95) (size 0.6) (drill 0.3) (layers "F.Cu" "B.Cu") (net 1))
 (via (at 153.2 55.95) (size 0.6) (drill 0.3) (layers "F.Cu" "B.Cu") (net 1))
 (segment (start 155.535 52.635) (end 155.535 51.7) (width 0.2) (layer "B.Cu") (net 1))
 (segment (start 168.235 61) (end 168.235 65.365) (width 0.2) (layer "B.Cu") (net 1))
 (segment (start 152.4 55.95) (end 153.2 55.95) (width 0.2) (layer "B.Cu") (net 1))
 (segment (start 168.235 65.365) (end 166.2 67.4) (width 0.2) (layer "B.Cu") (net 1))
 (segment (start 159.15 55.95) (end 158.85 55.95) (width 0.2) (layer "B.Cu") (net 1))
 (segment (start 151 54.8) (end 151.15 54.8) (width 0.2) (layer "B.Cu") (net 1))
 (segment (start 158.85 55.95) (end 155.535 52.635) (width 0.2) (layer "B.Cu") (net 1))
 (segment (start 166.965 61) (end 166.965 65.035) (width 0.2) (layer "B.Cu") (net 1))
 (segment (start 151.15 54.8) (end 151.2 54.75) (width 0.2) (layer "B.Cu") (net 1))
 (segment (start 151.2 54.75) (end 152.4 55.95) (width 0.2) (layer "B.Cu") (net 1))
 (segment (start 166.965 65.035) (end 165.2 66.8) (width 0.2) (layer "B.Cu") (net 1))
 (segment (start 147.1 63.65) (end 147.15 63.6) (width 0.2) (layer "F.Cu") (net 26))
 (segment (start 147.1 72) (end 147.1 63.65) (width 0.2) (layer "F.Cu") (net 26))
 (via (at 147.15 63.6) (size 0.6) (drill 0.3) (layers "F.Cu" "B.Cu") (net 26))
 (segment (start 147.4 63.35) (end 163.099999 63.35) (width 0.2) (layer "B.Cu") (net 26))
 (segment (start 163.099999 63.35) (end 164.425 62.024999) (width 0.2) (layer "B.Cu") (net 26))
 (segment (start 147.15 63.6) (end 147.4 63.35) (width 0.2) (layer "B.Cu") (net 26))
 (segment (start 164.425 62.024999) (end 164.425 61) (width 0.2) (layer "B.Cu") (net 26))
 (segment (start 146.1 72) (end 146.1 62.8) (width 0.2) (layer "F.Cu") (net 27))
 (segment (start 146.1 62.8) (end 146.15 62.75) (width 0.2) (layer "F.Cu") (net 27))
 (via (at 146.15 62.75) (size 0.6) (drill 0.3) (layers "F.Cu" "B.Cu") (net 27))
 (segment (start 161.801968 62.75) (end 163.155 61.396968) (width 0.2) (layer "B.Cu") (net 27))
 (segment (start 146.15 62.75) (end 161.801968 62.75) (width 0.2) (layer "B.Cu") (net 27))
 (segment (start 163.155 61.396968) (end 163.155 61) (width 0.2) (layer "B.Cu") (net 27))
 (segment (start 145.1 72) (end 145.1 61.95) (width 0.2) (layer "F.Cu") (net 28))
 (via (at 145.1 61.95) (size 0.6) (drill 0.3) (layers "F.Cu" "B.Cu") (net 28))
 (segment (start 160.955968 62.326) (end 161.885 61.396968) (width 0.2) (layer "B.Cu") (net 28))
 (segment (start 152.654032 62.326) (end 160.955968 62.326) (width 0.2) (layer "B.Cu") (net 28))
 (segment (start 145.1 61.95) (end 152.278032 61.95) (width 0.2) (layer "B.Cu") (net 28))
 (segment (start 152.278032 61.95) (end 152.654032 62.326) (width 0.2) (layer "B.Cu") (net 28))
 (segment (start 161.885 61.396968) (end 161.885 61) (width 0.2) (layer "B.Cu") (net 28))
 (segment (start 148.1 64.2) (end 148.15 64.15) (width 0.2) (layer "F.Cu") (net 25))
 (segment (start 148.1 72) (end 148.1 71.95) (width 0.2) (layer "F.Cu") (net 25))
 (segment (start 148.1 71.95) (end 148.1 64.2) (width 0.2) (layer "F.Cu") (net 25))
 (via (at 148.15 64.15) (size 0.6) (drill 0.3) (layers "F.Cu" "B.Cu") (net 25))
 (segment (start 162.941968 64.15) (end 165.695 61.396968) (width 0.2) (layer "B.Cu") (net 25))
 (segment (start 165.695 61.396968) (end 165.695 61) (width 0.2) (layer "B.Cu") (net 25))
 (segment (start 148.15 64.15) (end 162.941968 64.15) (width 0.2) (layer "B.Cu") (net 25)))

